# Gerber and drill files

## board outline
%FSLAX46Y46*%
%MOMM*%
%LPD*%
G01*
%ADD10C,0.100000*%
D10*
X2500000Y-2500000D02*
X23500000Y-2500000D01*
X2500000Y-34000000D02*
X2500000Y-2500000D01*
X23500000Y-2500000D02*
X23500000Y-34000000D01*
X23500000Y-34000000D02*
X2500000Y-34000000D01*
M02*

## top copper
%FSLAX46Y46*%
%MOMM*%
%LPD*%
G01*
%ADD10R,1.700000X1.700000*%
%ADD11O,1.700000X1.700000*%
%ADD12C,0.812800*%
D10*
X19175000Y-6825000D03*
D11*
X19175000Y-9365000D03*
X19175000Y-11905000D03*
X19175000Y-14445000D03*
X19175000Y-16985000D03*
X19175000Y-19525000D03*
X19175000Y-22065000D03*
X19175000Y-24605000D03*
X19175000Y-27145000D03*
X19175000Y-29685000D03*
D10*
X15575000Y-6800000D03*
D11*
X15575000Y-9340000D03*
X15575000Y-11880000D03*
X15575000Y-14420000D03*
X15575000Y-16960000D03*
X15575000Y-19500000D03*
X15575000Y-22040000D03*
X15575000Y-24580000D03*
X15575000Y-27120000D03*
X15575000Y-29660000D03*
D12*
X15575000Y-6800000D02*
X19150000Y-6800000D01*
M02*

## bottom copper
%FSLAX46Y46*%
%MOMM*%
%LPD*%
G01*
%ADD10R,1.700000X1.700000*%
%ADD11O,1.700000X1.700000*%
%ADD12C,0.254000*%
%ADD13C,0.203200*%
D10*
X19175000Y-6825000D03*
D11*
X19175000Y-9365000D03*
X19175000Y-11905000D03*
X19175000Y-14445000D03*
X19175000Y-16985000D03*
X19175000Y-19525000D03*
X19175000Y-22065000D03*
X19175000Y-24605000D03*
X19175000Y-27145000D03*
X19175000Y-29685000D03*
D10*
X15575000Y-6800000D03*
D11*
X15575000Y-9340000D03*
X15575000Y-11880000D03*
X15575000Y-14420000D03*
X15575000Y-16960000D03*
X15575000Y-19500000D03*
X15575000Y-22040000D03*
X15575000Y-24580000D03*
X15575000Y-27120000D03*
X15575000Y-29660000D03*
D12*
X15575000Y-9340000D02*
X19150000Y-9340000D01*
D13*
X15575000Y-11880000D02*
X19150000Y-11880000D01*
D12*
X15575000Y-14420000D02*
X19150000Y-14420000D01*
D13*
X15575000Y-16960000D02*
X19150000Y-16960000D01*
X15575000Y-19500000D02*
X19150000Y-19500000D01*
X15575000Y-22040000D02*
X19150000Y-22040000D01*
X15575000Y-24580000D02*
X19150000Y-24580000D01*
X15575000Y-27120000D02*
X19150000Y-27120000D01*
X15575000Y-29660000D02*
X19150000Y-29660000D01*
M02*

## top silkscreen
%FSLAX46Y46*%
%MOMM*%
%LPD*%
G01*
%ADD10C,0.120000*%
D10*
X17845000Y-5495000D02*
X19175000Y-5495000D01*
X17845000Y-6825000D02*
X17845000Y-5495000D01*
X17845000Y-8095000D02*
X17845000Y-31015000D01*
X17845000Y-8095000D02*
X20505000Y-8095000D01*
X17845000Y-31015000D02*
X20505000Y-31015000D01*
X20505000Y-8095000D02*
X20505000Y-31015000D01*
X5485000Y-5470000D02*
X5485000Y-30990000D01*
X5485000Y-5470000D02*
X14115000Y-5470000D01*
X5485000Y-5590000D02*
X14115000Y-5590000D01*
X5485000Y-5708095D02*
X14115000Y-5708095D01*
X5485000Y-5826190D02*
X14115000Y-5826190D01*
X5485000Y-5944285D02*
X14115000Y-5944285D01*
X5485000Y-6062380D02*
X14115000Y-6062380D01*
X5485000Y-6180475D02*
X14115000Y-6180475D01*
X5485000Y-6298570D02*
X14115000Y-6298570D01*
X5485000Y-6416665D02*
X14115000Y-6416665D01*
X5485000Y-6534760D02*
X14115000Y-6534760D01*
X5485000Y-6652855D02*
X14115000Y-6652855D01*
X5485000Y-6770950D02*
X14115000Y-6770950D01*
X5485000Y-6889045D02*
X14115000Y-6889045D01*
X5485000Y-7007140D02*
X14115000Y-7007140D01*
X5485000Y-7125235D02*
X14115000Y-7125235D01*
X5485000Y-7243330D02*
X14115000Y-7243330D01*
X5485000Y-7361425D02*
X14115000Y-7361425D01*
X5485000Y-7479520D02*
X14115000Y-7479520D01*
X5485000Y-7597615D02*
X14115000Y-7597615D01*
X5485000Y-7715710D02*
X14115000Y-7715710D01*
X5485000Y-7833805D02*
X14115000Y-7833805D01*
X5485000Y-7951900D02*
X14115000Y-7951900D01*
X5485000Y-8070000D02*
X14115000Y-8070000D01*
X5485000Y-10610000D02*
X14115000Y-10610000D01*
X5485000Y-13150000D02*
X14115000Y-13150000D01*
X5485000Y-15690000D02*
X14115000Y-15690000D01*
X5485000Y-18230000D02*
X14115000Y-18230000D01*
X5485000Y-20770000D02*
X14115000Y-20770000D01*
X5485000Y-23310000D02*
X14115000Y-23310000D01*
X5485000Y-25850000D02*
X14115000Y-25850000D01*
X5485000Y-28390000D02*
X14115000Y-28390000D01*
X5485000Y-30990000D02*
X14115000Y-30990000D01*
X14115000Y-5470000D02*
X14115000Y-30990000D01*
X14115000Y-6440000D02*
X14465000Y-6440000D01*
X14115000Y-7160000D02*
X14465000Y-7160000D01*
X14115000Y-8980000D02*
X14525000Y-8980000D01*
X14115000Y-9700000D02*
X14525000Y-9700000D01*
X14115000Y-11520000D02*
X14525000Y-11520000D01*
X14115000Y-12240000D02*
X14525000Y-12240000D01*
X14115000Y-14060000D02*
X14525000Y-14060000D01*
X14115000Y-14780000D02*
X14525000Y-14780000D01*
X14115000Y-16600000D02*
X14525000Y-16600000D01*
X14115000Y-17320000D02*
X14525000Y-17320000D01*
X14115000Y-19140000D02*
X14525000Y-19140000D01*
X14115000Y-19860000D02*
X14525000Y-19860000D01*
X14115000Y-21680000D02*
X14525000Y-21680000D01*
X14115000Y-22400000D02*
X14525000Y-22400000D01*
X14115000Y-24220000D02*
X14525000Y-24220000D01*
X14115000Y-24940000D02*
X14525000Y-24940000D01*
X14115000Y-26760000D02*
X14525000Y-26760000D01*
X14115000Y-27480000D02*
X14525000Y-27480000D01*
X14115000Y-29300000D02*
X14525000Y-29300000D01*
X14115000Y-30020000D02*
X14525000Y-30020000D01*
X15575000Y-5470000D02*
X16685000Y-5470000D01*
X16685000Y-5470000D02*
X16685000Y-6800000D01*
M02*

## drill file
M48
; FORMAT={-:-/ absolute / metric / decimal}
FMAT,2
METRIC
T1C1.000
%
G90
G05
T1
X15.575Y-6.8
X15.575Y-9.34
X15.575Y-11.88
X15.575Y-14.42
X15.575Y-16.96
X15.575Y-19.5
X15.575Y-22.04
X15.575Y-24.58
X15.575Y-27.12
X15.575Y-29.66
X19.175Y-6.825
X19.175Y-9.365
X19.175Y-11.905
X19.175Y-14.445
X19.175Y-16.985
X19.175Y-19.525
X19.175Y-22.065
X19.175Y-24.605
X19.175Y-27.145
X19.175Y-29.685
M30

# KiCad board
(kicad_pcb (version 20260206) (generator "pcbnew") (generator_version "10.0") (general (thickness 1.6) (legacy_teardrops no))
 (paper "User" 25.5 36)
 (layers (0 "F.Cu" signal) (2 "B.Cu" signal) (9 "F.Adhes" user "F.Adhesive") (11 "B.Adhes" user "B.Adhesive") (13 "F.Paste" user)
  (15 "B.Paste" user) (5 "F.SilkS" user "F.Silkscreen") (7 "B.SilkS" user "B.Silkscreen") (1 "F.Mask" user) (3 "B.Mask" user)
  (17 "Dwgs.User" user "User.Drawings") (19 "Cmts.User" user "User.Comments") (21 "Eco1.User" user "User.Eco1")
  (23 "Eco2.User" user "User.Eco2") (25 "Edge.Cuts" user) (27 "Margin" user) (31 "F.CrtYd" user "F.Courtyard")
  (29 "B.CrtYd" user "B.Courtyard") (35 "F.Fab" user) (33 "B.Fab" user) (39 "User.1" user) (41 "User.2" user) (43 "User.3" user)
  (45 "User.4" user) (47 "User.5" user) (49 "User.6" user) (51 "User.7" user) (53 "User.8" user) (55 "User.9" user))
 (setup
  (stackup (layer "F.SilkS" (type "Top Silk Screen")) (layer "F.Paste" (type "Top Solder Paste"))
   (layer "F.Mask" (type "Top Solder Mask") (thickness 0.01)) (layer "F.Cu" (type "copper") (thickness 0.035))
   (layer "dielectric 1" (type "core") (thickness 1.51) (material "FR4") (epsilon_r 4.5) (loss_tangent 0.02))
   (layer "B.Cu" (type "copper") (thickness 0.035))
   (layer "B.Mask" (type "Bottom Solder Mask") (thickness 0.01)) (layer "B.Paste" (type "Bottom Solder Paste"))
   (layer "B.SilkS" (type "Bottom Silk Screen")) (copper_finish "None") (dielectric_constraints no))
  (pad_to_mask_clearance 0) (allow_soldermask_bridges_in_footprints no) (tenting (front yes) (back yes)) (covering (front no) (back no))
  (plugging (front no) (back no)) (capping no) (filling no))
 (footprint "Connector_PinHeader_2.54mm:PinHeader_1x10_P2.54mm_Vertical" (layer "F.Cu") (at 19.175 6.825)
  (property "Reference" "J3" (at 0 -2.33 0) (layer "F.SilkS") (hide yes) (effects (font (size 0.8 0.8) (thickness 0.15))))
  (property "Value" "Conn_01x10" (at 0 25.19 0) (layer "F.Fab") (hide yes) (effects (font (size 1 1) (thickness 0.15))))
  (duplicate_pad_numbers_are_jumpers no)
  (fp_line (start -1.33 -1.33) (end 0 -1.33) (stroke (width 0.12) (type solid)) (layer "F.SilkS"))
  (fp_line (start -1.33 0) (end -1.33 -1.33) (stroke (width 0.12) (type solid)) (layer "F.SilkS"))
  (fp_line (start -1.33 1.27) (end -1.33 24.19) (stroke (width 0.12) (type solid)) (layer "F.SilkS"))
  (fp_line (start -1.33 1.27) (end 1.33 1.27) (stroke (width 0.12) (type solid)) (layer "F.SilkS"))
  (fp_line (start -1.33 24.19) (end 1.33 24.19) (stroke (width 0.12) (type solid)) (layer "F.SilkS"))
  (fp_line (start 1.33 1.27) (end 1.33 24.19) (stroke (width 0.12) (type solid)) (layer "F.SilkS"))
  (pad "1" thru_hole rect (at 0 0) (size 1.7 1.7) (drill 1) (layers "*.Cu" "*.Mask") (remove_unused_layers no) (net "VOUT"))
  (pad "2" thru_hole oval (at 0 2.54) (size 1.7 1.7) (drill 1) (layers "*.Cu" "*.Mask") (remove_unused_layers no) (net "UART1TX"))
  (pad "3" thru_hole oval (at 0 5.08) (size 1.7 1.7) (drill 1) (layers "*.Cu" "*.Mask") (remove_unused_layers no) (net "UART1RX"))
  (pad "4" thru_hole oval (at 0 7.62) (size 1.7 1.7) (drill 1) (layers "*.Cu" "*.Mask") (remove_unused_layers no) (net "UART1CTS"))
  (pad "5" thru_hole oval (at 0 10.16) (size 1.7 1.7) (drill 1) (layers "*.Cu" "*.Mask") (remove_unused_layers no) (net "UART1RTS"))
  (pad "6" thru_hole oval (at 0 12.7) (size 1.7 1.7) (drill 1) (layers "*.Cu" "*.Mask") (remove_unused_layers no) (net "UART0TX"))
  (pad "7" thru_hole oval (at 0 15.24) (size 1.7 1.7) (drill 1) (layers "*.Cu" "*.Mask") (remove_unused_layers no) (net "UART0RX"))
  (pad "8" thru_hole oval (at 0 17.78) (size 1.7 1.7) (drill 1) (layers "*.Cu" "*.Mask") (remove_unused_layers no) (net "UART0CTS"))
  (pad "9" thru_hole oval (at 0 20.32) (size 1.7 1.7) (drill 1) (layers "*.Cu" "*.Mask") (remove_unused_layers no) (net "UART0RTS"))
  (pad "10" thru_hole oval (at 0 22.86) (size 1.7 1.7) (drill 1) (layers "*.Cu" "*.Mask") (remove_unused_layers no) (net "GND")))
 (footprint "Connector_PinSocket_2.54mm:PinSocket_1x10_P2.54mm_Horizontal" (layer "F.Cu") (at 15.575 6.8)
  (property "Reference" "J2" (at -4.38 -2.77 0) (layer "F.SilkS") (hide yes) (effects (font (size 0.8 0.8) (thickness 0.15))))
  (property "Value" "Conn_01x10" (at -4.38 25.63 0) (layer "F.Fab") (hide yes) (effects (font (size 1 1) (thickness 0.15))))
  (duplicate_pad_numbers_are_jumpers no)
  (fp_line (start -10.09 -1.33) (end -10.09 24.19) (stroke (width 0.12) (type solid)) (layer "F.SilkS"))
  (fp_line (start -10.09 -1.33) (end -1.46 -1.33) (stroke (width 0.12) (type solid)) (layer "F.SilkS"))
  (fp_line (start -10.09 -1.21) (end -1.46 -1.21) (stroke (width 0.12) (type solid)) (layer "F.SilkS"))
  (fp_line (start -10.09 -1.091905) (end -1.46 -1.091905) (stroke (width 0.12) (type solid)) (layer "F.SilkS"))
  (fp_line (start -10.09 -0.97381) (end -1.46 -0.97381) (stroke (width 0.12) (type solid)) (layer "F.SilkS"))
  (fp_line (start -10.09 -0.855715) (end -1.46 -0.855715) (stroke (width 0.12) (type solid)) (layer "F.SilkS"))
  (fp_line (start -10.09 -0.73762) (end -1.46 -0.73762) (stroke (width 0.12) (type solid)) (layer "F.SilkS"))
  (fp_line (start -10.09 -0.619525) (end -1.46 -0.619525) (stroke (width 0.12) (type solid)) (layer "F.SilkS"))
  (fp_line (start -10.09 -0.50143) (end -1.46 -0.50143) (stroke (width 0.12) (type solid)) (layer "F.SilkS"))
  (fp_line (start -10.09 -0.383335) (end -1.46 -0.383335) (stroke (width 0.12) (type solid)) (layer "F.SilkS"))
  (fp_line (start -10.09 -0.26524) (end -1.46 -0.26524) (stroke (width 0.12) (type solid)) (layer "F.SilkS"))
  (fp_line (start -10.09 -0.147145) (end -1.46 -0.147145) (stroke (width 0.12) (type solid)) (layer "F.SilkS"))
  (fp_line (start -10.09 -0.02905) (end -1.46 -0.02905) (stroke (width 0.12) (type solid)) (layer "F.SilkS"))
  (fp_line (start -10.09 0.089045) (end -1.46 0.089045) (stroke (width 0.12) (type solid)) (layer "F.SilkS"))
  (fp_line (start -10.09 0.20714) (end -1.46 0.20714) (stroke (width 0.12) (type solid)) (layer "F.SilkS"))
  (fp_line (start -10.09 0.325235) (end -1.46 0.325235) (stroke (width 0.12) (type solid)) (layer "F.SilkS"))
  (fp_line (start -10.09 0.44333) (end -1.46 0.44333) (stroke (width 0.12) (type solid)) (layer "F.SilkS"))
  (fp_line (start -10.09 0.561425) (end -1.46 0.561425) (stroke (width 0.12) (type solid)) (layer "F.SilkS"))
  (fp_line (start -10.09 0.67952) (end -1.46 0.67952) (stroke (width 0.12) (type solid)) (layer "F.SilkS"))
  (fp_line (start -10.09 0.797615) (end -1.46 0.797615) (stroke (width 0.12) (type solid)) (layer "F.SilkS"))
  (fp_line (start -10.09 0.91571) (end -1.46 0.91571) (stroke (width 0.12) (type solid)) (layer "F.SilkS"))
  (fp_line (start -10.09 1.033805) (end -1.46 1.033805) (stroke (width 0.12) (type solid)) (layer "F.SilkS"))
  (fp_line (start -10.09 1.1519) (end -1.46 1.1519) (stroke (width 0.12) (type solid)) (layer "F.SilkS"))
  (fp_line (start -10.09 1.27) (end -1.46 1.27) (stroke (width 0.12) (type solid)) (layer "F.SilkS"))
  (fp_line (start -10.09 3.81) (end -1.46 3.81) (stroke (width 0.12) (type solid)) (layer "F.SilkS"))
  (fp_line (start -10.09 6.35) (end -1.46 6.35) (stroke (width 0.12) (type solid)) (layer "F.SilkS"))
  (fp_line (start -10.09 8.89) (end -1.46 8.89) (stroke (width 0.12) (type solid)) (layer "F.SilkS"))
  (fp_line (start -10.09 11.43) (end -1.46 11.43) (stroke (width 0.12) (type solid)) (layer "F.SilkS"))
  (fp_line (start -10.09 13.97) (end -1.46 13.97) (stroke (width 0.12) (type solid)) (layer "F.SilkS"))
  (fp_line (start -10.09 16.51) (end -1.46 16.51) (stroke (width 0.12) (type solid)) (layer "F.SilkS"))
  (fp_line (start -10.09 19.05) (end -1.46 19.05) (stroke (width 0.12) (type solid)) (layer "F.SilkS"))
  (fp_line (start -10.09 21.59) (end -1.46 21.59) (stroke (width 0.12) (type solid)) (layer "F.SilkS"))
  (fp_line (start -10.09 24.19) (end -1.46 24.19) (stroke (width 0.12) (type solid)) (layer "F.SilkS"))
  (fp_line (start -1.46 -1.33) (end -1.46 24.19) (stroke (width 0.12) (type solid)) (layer "F.SilkS"))
  (fp_line (start -1.46 -0.36) (end -1.11 -0.36) (stroke (width 0.12) (type solid)) (layer "F.SilkS"))
  (fp_line (start -1.46 0.36) (end -1.11 0.36) (stroke (width 0.12) (type solid)) (layer "F.SilkS"))
  (fp_line (start -1.46 2.18) (end -1.05 2.18) (stroke (width 0.12) (type solid)) (layer "F.SilkS"))
  (fp_line (start -1.46 2.9) (end -1.05 2.9) (stroke (width 0.12) (type solid)) (layer "F.SilkS"))
  (fp_line (start -1.46 4.72) (end -1.05 4.72) (stroke (width 0.12) (type solid)) (layer "F.SilkS"))
  (fp_line (start -1.46 5.44) (end -1.05 5.44) (stroke (width 0.12) (type solid)) (layer "F.SilkS"))
  (fp_line (start -1.46 7.26) (end -1.05 7.26) (stroke (width 0.12) (type solid)) (layer "F.SilkS"))
  (fp_line (start -1.46 7.98) (end -1.05 7.98) (stroke (width 0.12) (type solid)) (layer "F.SilkS"))
  (fp_line (start -1.46 9.8) (end -1.05 9.8) (stroke (width 0.12) (type solid)) (layer "F.SilkS"))
  (fp_line (start -1.46 10.52) (end -1.05 10.52) (stroke (width 0.12) (type solid)) (layer "F.SilkS"))
  (fp_line (start -1.46 12.34) (end -1.05 12.34) (stroke (width 0.12) (type solid)) (layer "F.SilkS"))
  (fp_line (start -1.46 13.06) (end -1.05 13.06) (stroke (width 0.12) (type solid)) (layer "F.SilkS"))
  (fp_line (start -1.46 14.88) (end -1.05 14.88) (stroke (width 0.12) (type solid)) (layer "F.SilkS"))
  (fp_line (start -1.46 15.6) (end -1.05 15.6) (stroke (width 0.12) (type solid)) (layer "F.SilkS"))
  (fp_line (start -1.46 17.42) (end -1.05 17.42) (stroke (width 0.12) (type solid)) (layer "F.SilkS"))
  (fp_line (start -1.46 18.14) (end -1.05 18.14) (stroke (width 0.12) (type solid)) (layer "F.SilkS"))
  (fp_line (start -1.46 19.96) (end -1.05 19.96) (stroke (width 0.12) (type solid)) (layer "F.SilkS"))
  (fp_line (start -1.46 20.68) (end -1.05 20.68) (stroke (width 0.12) (type solid)) (layer "F.SilkS"))
  (fp_line (start -1.46 22.5) (end -1.05 22.5) (stroke (width 0.12) (type solid)) (layer "F.SilkS"))
  (fp_line (start -1.46 23.22) (end -1.05 23.22) (stroke (width 0.12) (type solid)) (layer "F.SilkS"))
  (fp_line (start 0 -1.33) (end 1.11 -1.33) (stroke (width 0.12) (type solid)) (layer "F.SilkS"))
  (fp_line (start 1.11 -1.33) (end 1.11 0) (stroke (width 0.12) (type solid)) (layer "F.SilkS"))
  (pad "1" thru_hole rect (at 0 0) (size 1.7 1.7) (drill 1) (layers "*.Cu" "*.Mask") (remove_unused_layers no) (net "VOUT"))
  (pad "2" thru_hole oval (at 0 2.54) (size 1.7 1.7) (drill 1) (layers "*.Cu" "*.Mask") (remove_unused_layers no) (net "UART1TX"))
  (pad "3" thru_hole oval (at 0 5.08) (size 1.7 1.7) (drill 1) (layers "*.Cu" "*.Mask") (remove_unused_layers no) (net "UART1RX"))
  (pad "4" thru_hole oval (at 0 7.62) (size 1.7 1.7) (drill 1) (layers "*.Cu" "*.Mask") (remove_unused_layers no) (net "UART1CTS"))
  (pad "5" thru_hole oval (at 0 10.16) (size 1.7 1.7) (drill 1) (layers "*.Cu" "*.Mask") (remove_unused_layers no) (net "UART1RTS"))
  (pad "6" thru_hole oval (at 0 12.7) (size 1.7 1.7) (drill 1) (layers "*.Cu" "*.Mask") (remove_unused_layers no) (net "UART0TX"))
  (pad "7" thru_hole oval (at 0 15.24) (size 1.7 1.7) (drill 1) (layers "*.Cu" "*.Mask") (remove_unused_layers no) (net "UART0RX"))
  (pad "8" thru_hole oval (at 0 17.78) (size 1.7 1.7) (drill 1) (layers "*.Cu" "*.Mask") (remove_unused_layers no) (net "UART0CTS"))
  (pad "9" thru_hole oval (at 0 20.32) (size 1.7 1.7) (drill 1) (layers "*.Cu" "*.Mask") (remove_unused_layers no) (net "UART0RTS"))
  (pad "10" thru_hole oval (at 0 22.86) (size 1.7 1.7) (drill 1) (layers "*.Cu" "*.Mask") (remove_unused_layers no) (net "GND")))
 (gr_line (start 2.5 2.5) (end 23.5 2.5) (stroke (width 0.1) (type default)) (layer "Edge.Cuts"))
 (gr_line (start 2.5 34) (end 2.5 2.5) (stroke (width 0.1) (type default)) (layer "Edge.Cuts"))
 (gr_line (start 23.5 2.5) (end 23.5 34) (stroke (width 0.1) (type default)) (layer "Edge.Cuts"))
 (gr_line (start 23.5 34) (end 2.5 34) (stroke (width 0.1) (type default)) (layer "Edge.Cuts"))
 (segment (start 15.575 6.8) (end 19.15 6.8) (width 0.8128) (layer "F.Cu") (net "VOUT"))
 (segment (start 15.575 9.34) (end 19.15 9.34) (width 0.254) (layer "B.Cu") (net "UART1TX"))
 (segment (start 15.575 11.88) (end 19.15 11.88) (width 0.2032) (layer "B.Cu") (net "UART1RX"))
 (segment (start 15.575 14.42) (end 19.15 14.42) (width 0.254) (layer "B.Cu") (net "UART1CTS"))
 (segment (start 15.575 16.96) (end 19.15 16.96) (width 0.2032) (layer "B.Cu") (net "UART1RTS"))
 (segment (start 15.575 19.5) (end 19.15 19.5) (width 0.2032) (layer "B.Cu") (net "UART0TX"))
 (segment (start 15.575 22.04) (end 19.15 22.04) (width 0.2032) (layer "B.Cu") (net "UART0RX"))
 (segment (start 15.575 24.58) (end 19.15 24.58) (width 0.2032) (layer "B.Cu") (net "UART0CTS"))
 (segment (start 15.575 27.12) (end 19.15 27.12) (width 0.2032) (layer "B.Cu") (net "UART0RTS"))
 (segment (start 15.575 29.66) (end 19.15 29.66) (width 0.2032) (layer "B.Cu") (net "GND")))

